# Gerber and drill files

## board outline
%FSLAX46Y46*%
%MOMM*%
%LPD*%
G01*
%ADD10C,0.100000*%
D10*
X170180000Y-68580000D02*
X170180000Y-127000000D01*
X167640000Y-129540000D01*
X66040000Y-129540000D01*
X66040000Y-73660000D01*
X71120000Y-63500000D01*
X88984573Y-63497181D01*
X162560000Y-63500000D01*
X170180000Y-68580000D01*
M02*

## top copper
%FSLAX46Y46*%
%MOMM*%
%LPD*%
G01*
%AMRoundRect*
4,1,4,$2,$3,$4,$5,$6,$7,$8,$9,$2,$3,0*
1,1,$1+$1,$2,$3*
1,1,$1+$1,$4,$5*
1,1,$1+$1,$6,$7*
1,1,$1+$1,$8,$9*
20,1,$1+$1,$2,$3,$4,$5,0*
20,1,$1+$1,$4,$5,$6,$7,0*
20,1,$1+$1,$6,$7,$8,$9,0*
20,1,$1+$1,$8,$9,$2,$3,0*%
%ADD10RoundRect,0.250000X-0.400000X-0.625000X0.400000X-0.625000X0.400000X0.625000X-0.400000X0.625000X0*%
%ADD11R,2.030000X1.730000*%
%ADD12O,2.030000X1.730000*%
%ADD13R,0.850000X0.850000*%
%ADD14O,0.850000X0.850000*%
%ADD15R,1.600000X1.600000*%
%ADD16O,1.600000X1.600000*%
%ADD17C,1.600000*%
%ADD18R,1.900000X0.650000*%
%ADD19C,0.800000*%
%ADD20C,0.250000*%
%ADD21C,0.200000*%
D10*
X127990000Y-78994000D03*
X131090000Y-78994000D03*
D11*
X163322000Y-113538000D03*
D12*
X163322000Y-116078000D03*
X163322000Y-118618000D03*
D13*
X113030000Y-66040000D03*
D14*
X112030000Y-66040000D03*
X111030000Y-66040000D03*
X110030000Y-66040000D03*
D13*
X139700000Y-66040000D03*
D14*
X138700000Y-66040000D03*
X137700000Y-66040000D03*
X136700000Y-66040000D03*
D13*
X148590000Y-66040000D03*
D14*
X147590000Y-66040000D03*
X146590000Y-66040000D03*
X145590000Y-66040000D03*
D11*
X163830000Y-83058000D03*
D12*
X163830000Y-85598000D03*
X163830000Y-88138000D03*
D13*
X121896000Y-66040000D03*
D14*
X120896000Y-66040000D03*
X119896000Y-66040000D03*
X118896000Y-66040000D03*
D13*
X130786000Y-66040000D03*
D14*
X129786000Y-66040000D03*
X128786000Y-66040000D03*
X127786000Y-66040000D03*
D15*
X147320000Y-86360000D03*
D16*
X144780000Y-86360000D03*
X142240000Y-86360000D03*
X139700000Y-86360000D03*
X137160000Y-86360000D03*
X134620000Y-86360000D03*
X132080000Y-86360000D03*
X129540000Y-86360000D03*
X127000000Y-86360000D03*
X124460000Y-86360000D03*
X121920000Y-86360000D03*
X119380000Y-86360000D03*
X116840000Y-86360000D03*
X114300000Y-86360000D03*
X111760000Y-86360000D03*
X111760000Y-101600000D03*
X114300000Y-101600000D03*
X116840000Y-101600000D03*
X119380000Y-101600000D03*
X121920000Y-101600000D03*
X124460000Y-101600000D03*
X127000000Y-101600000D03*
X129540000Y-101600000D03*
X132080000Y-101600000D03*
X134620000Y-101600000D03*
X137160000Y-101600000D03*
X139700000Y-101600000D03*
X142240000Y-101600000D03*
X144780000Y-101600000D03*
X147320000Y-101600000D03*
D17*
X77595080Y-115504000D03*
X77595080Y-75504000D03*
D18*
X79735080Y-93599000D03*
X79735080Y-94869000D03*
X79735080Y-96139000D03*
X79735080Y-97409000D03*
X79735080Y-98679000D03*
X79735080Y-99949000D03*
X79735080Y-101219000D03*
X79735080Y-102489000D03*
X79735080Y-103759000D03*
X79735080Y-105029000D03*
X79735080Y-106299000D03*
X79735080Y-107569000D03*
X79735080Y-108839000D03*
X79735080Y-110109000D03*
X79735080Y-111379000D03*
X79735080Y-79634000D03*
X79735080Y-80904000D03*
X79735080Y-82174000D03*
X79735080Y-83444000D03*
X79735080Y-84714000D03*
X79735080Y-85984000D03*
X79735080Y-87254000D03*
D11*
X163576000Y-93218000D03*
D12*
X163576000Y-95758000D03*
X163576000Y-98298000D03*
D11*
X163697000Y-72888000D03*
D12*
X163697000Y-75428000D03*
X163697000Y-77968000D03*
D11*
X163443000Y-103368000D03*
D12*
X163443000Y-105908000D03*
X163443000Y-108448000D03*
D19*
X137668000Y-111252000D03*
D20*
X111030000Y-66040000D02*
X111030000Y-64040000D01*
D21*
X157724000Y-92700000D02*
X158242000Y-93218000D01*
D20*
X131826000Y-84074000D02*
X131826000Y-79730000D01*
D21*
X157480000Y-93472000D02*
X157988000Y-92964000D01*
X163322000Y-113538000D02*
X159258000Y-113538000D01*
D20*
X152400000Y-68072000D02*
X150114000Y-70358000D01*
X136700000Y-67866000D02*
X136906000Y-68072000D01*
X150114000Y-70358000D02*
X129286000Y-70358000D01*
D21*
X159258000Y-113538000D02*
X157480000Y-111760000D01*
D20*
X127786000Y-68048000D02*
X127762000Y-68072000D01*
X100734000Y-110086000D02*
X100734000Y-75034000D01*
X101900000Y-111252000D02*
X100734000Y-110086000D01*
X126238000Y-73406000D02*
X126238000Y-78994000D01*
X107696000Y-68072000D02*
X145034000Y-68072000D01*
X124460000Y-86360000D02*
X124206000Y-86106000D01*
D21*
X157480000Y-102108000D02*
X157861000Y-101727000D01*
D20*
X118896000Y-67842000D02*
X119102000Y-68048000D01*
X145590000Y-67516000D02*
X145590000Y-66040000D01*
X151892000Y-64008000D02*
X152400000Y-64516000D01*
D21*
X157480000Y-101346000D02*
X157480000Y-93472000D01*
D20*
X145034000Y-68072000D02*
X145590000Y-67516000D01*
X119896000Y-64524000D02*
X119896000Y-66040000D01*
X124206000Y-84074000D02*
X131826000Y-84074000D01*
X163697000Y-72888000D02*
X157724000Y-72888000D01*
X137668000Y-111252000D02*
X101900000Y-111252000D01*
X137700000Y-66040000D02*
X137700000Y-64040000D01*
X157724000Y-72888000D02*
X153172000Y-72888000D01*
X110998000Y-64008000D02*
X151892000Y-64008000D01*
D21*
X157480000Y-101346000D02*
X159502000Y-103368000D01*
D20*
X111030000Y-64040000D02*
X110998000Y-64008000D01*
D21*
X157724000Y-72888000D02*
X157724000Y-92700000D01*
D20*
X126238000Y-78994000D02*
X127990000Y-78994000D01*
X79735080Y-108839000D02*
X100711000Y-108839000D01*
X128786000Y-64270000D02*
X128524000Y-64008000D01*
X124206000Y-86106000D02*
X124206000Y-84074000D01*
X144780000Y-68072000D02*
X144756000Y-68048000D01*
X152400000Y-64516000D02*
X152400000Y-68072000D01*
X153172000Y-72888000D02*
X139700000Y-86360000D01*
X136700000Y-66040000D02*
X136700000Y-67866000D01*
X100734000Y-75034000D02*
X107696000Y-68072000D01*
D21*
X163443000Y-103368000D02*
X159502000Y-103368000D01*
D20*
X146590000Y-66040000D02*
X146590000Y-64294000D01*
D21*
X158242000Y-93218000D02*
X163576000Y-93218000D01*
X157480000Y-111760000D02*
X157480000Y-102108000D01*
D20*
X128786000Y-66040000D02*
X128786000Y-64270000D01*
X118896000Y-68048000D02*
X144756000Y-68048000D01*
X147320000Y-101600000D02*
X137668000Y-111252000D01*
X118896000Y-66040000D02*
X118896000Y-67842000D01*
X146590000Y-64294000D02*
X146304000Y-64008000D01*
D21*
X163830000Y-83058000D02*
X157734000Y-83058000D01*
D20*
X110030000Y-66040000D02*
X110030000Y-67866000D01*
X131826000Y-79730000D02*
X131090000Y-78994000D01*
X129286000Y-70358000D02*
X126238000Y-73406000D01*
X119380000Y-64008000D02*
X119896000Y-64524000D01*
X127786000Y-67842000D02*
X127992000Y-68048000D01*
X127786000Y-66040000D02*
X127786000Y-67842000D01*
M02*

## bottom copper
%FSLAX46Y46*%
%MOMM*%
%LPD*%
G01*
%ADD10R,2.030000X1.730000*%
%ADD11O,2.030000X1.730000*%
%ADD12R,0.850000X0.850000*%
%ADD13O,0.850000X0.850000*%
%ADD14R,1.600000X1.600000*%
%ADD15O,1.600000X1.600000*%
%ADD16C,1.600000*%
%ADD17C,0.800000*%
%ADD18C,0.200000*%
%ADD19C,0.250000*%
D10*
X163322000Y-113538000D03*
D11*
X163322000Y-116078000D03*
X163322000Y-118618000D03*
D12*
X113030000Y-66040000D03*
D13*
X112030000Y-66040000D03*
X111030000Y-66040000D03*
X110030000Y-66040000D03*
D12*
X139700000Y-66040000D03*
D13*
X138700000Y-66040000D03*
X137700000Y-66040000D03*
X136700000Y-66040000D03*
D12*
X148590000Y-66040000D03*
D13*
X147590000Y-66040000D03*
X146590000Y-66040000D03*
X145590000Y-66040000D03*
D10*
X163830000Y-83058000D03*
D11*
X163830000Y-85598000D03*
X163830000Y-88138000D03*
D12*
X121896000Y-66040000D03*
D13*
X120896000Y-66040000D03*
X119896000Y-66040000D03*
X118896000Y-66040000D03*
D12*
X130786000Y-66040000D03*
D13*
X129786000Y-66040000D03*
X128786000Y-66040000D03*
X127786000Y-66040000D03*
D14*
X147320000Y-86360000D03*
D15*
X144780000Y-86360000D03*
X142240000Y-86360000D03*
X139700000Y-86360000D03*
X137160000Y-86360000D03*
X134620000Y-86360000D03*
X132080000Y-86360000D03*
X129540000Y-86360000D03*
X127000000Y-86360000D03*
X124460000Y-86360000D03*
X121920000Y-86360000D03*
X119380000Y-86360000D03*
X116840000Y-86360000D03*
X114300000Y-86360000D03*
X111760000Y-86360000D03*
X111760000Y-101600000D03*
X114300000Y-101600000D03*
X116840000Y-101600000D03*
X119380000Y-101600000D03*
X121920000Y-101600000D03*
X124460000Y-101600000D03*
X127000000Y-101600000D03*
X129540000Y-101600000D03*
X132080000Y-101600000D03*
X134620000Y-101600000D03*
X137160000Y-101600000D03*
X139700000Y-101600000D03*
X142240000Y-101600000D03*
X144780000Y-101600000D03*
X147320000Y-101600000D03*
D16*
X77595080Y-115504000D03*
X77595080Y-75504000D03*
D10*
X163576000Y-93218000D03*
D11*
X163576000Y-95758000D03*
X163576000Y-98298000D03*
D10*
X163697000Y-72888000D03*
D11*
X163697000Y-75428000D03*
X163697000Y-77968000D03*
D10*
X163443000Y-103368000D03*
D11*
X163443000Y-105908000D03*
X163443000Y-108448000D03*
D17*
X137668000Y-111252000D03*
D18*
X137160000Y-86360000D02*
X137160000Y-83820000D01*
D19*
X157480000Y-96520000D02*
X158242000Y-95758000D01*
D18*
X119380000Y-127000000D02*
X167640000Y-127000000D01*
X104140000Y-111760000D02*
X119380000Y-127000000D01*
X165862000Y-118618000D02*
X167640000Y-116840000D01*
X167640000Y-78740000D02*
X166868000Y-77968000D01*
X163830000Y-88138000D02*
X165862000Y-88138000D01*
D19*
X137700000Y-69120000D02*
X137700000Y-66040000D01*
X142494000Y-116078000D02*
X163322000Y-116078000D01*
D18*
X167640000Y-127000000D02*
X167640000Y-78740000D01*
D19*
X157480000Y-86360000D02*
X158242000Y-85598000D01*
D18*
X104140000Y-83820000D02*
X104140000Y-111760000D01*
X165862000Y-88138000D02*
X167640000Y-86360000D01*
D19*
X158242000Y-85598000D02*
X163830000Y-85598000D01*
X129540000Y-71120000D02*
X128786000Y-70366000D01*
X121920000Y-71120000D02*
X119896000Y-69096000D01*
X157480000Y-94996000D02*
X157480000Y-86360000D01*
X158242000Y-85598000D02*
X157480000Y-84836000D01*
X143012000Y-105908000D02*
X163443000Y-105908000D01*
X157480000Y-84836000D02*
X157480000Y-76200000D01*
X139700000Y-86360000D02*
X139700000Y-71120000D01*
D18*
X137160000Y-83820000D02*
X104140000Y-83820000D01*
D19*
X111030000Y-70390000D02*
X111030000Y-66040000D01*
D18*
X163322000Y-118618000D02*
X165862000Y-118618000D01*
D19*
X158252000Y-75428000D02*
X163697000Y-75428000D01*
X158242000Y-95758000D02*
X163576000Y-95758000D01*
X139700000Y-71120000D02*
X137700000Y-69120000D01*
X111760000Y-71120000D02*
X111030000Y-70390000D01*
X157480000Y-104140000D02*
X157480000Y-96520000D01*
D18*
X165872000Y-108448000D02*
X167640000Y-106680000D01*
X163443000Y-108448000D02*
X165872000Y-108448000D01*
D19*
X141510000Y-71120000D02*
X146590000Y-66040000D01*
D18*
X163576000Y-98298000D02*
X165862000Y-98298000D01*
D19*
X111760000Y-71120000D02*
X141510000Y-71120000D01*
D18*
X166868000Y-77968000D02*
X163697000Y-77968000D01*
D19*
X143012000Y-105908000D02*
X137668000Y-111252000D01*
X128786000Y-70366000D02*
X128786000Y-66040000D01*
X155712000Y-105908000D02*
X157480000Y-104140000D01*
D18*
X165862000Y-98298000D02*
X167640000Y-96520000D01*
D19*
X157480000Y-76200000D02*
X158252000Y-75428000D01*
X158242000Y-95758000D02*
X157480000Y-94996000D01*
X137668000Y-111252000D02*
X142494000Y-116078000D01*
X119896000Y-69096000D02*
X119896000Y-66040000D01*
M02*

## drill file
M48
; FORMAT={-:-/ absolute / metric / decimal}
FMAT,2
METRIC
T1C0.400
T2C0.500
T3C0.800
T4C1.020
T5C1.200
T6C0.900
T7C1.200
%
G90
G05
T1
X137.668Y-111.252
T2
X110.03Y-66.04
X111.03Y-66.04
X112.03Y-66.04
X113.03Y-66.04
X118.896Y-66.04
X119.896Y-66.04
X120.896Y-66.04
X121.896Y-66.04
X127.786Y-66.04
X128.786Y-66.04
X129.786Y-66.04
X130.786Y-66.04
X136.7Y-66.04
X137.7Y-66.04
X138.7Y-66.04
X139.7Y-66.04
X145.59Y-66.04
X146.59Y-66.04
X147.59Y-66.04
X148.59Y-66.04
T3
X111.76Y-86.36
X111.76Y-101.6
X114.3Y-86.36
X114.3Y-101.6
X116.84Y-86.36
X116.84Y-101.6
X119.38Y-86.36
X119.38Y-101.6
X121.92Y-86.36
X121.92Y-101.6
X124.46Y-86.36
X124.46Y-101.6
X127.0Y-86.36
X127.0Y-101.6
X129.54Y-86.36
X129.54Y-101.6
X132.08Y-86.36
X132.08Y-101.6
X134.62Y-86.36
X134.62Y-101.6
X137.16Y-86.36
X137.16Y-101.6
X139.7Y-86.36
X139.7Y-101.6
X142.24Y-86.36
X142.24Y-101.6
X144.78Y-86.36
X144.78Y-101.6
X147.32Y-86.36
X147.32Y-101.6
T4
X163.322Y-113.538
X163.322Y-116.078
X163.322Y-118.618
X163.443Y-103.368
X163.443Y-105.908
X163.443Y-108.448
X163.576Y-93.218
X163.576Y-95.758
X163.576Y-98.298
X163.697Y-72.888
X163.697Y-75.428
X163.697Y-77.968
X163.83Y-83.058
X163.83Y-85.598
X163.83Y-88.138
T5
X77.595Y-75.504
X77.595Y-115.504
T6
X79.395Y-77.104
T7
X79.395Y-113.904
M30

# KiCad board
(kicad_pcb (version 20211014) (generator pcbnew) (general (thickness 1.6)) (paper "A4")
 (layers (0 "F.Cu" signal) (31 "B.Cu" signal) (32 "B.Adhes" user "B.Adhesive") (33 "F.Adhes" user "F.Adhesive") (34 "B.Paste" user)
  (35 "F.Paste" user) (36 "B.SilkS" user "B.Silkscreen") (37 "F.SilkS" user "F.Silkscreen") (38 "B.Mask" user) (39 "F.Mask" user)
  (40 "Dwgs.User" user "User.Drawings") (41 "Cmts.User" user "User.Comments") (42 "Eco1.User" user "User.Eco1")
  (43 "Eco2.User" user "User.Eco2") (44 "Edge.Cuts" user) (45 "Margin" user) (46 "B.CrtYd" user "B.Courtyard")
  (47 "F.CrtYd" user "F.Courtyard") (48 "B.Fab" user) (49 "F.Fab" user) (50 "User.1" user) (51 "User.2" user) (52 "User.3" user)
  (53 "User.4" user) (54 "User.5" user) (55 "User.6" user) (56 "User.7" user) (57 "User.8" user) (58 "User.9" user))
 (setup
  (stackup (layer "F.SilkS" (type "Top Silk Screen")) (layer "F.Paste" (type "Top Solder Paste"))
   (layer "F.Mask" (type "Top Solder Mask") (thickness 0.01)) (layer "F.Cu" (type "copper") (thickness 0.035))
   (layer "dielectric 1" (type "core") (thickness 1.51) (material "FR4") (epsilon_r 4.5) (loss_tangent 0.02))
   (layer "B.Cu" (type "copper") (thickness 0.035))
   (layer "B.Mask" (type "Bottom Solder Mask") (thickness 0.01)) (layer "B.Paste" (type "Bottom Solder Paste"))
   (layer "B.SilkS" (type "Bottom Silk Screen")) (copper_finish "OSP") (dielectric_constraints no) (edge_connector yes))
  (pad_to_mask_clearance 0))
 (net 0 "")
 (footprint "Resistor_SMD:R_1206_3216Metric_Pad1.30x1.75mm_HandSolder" (layer "F.Cu") (at 129.54 78.994)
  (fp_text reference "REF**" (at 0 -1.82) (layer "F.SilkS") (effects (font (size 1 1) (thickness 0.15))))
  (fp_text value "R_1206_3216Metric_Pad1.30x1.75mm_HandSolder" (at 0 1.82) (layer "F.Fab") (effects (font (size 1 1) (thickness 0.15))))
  (pad "1" smd roundrect (at -1.55 0) (size 1.3 1.75) (layers "F.Cu" "F.Paste" "F.Mask") (roundrect_rratio 0.1923076923))
  (pad "2" smd roundrect (at 1.55 0) (size 1.3 1.75) (layers "F.Cu" "F.Paste" "F.Mask") (roundrect_rratio 0.1923076923)))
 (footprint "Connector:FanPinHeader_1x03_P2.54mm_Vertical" (layer "F.Cu") (at 163.322 113.538 -90)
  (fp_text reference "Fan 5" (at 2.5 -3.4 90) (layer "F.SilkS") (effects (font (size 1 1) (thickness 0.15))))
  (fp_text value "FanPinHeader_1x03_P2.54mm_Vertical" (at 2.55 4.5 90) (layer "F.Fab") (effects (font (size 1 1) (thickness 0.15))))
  (pad "1" thru_hole rect (at 0 0) (size 2.03 1.73) (drill 1.02) (layers *.Cu *.Mask))
  (pad "2" thru_hole oval (at 2.54 0) (size 2.03 1.73) (drill 1.02) (layers *.Cu *.Mask))
  (pad "3" thru_hole oval (at 5.08 0) (size 2.03 1.73) (drill 1.02) (layers *.Cu *.Mask)))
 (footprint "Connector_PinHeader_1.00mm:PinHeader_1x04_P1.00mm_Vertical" (layer "F.Cu") (at 113.03 66.04 -90)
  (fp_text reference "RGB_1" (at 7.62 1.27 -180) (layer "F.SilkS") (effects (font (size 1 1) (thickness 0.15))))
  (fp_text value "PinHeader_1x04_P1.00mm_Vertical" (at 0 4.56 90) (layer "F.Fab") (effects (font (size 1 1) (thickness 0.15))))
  (pad "1" thru_hole rect (at 0 0 270) (size 0.85 0.85) (drill 0.5) (layers *.Cu *.Mask))
  (pad "2" thru_hole oval (at 0 1 270) (size 0.85 0.85) (drill 0.5) (layers *.Cu *.Mask))
  (pad "3" thru_hole oval (at 0 2 270) (size 0.85 0.85) (drill 0.5) (layers *.Cu *.Mask))
  (pad "4" thru_hole oval (at 0 3 270) (size 0.85 0.85) (drill 0.5) (layers *.Cu *.Mask)))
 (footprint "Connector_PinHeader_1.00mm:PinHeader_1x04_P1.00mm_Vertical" (layer "F.Cu") (at 139.7 66.04 -90)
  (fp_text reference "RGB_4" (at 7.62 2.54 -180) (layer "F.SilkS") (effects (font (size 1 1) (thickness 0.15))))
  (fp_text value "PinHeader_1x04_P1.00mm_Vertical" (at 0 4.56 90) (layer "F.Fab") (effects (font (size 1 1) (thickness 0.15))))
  (pad "1" thru_hole rect (at 0 0 270) (size 0.85 0.85) (drill 0.5) (layers *.Cu *.Mask))
  (pad "2" thru_hole oval (at 0 1 270) (size 0.85 0.85) (drill 0.5) (layers *.Cu *.Mask))
  (pad "3" thru_hole oval (at 0 2 270) (size 0.85 0.85) (drill 0.5) (layers *.Cu *.Mask))
  (pad "4" thru_hole oval (at 0 3 270) (size 0.85 0.85) (drill 0.5) (layers *.Cu *.Mask)))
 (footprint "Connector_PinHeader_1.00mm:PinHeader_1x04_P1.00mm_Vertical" (layer "F.Cu") (at 148.59 66.04 -90)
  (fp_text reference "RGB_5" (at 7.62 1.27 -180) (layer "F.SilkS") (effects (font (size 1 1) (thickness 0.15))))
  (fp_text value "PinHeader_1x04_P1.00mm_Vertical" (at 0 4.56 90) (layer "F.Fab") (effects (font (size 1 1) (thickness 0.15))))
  (pad "1" thru_hole rect (at 0 0 270) (size 0.85 0.85) (drill 0.5) (layers *.Cu *.Mask))
  (pad "2" thru_hole oval (at 0 1 270) (size 0.85 0.85) (drill 0.5) (layers *.Cu *.Mask))
  (pad "3" thru_hole oval (at 0 2 270) (size 0.85 0.85) (drill 0.5) (layers *.Cu *.Mask))
  (pad "4" thru_hole oval (at 0 3 270) (size 0.85 0.85) (drill 0.5) (layers *.Cu *.Mask)))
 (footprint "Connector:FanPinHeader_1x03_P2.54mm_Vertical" (layer "F.Cu") (at 163.83 83.058 -90)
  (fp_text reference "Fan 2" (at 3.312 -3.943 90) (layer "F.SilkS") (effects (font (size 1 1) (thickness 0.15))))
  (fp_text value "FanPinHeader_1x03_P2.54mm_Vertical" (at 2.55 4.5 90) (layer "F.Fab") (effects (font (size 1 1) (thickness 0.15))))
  (pad "1" thru_hole rect (at 0 0) (size 2.03 1.73) (drill 1.02) (layers *.Cu *.Mask))
  (pad "2" thru_hole oval (at 2.54 0) (size 2.03 1.73) (drill 1.02) (layers *.Cu *.Mask))
  (pad "3" thru_hole oval (at 5.08 0) (size 2.03 1.73) (drill 1.02) (layers *.Cu *.Mask)))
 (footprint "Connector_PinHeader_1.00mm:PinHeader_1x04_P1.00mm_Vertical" (layer "F.Cu") (at 121.896 66.04 -90)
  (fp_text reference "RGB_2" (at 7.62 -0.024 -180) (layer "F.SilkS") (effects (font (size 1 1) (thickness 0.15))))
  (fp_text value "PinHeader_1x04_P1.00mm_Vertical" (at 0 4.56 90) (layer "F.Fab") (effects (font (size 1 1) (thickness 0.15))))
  (pad "1" thru_hole rect (at 0 0 270) (size 0.85 0.85) (drill 0.5) (layers *.Cu *.Mask))
  (pad "2" thru_hole oval (at 0 1 270) (size 0.85 0.85) (drill 0.5) (layers *.Cu *.Mask))
  (pad "3" thru_hole oval (at 0 2 270) (size 0.85 0.85) (drill 0.5) (layers *.Cu *.Mask))
  (pad "4" thru_hole oval (at 0 3 270) (size 0.85 0.85) (drill 0.5) (layers *.Cu *.Mask)))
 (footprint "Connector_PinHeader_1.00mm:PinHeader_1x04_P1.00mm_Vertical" (layer "F.Cu") (at 130.786 66.04 -90)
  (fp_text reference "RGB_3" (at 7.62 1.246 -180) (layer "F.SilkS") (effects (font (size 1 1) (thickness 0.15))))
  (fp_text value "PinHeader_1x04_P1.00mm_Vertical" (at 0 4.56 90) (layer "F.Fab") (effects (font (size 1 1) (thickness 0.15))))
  (pad "1" thru_hole rect (at 0 0 270) (size 0.85 0.85) (drill 0.5) (layers *.Cu *.Mask))
  (pad "2" thru_hole oval (at 0 1 270) (size 0.85 0.85) (drill 0.5) (layers *.Cu *.Mask))
  (pad "3" thru_hole oval (at 0 2 270) (size 0.85 0.85) (drill 0.5) (layers *.Cu *.Mask))
  (pad "4" thru_hole oval (at 0 3 270) (size 0.85 0.85) (drill 0.5) (layers *.Cu *.Mask)))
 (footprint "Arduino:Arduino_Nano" (layer "F.Cu") (at 147.32 86.36 -90)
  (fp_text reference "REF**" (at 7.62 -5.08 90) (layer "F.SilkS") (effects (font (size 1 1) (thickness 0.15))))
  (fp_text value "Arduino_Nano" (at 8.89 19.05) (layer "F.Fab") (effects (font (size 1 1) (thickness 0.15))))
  (pad "1" thru_hole rect locked (at 0 0 270) (size 1.6 1.6) (drill 0.8) (layers *.Cu *.Mask))
  (pad "2" thru_hole oval locked (at 0 2.54 270) (size 1.6 1.6) (drill 0.8) (layers *.Cu *.Mask))
  (pad "3" thru_hole oval locked (at 0 5.08 270) (size 1.6 1.6) (drill 0.8) (layers *.Cu *.Mask))
  (pad "4" thru_hole oval locked (at 0 7.62 270) (size 1.6 1.6) (drill 0.8) (layers *.Cu *.Mask))
  (pad "5" thru_hole oval locked (at 0 10.16 270) (size 1.6 1.6) (drill 0.8) (layers *.Cu *.Mask))
  (pad "6" thru_hole oval locked (at 0 12.7 270) (size 1.6 1.6) (drill 0.8) (layers *.Cu *.Mask))
  (pad "7" thru_hole oval locked (at 0 15.24 270) (size 1.6 1.6) (drill 0.8) (layers *.Cu *.Mask))
  (pad "8" thru_hole oval locked (at 0 17.78 270) (size 1.6 1.6) (drill 0.8) (layers *.Cu *.Mask))
  (pad "9" thru_hole oval locked (at 0 20.32 270) (size 1.6 1.6) (drill 0.8) (layers *.Cu *.Mask))
  (pad "10" thru_hole oval locked (at 0 22.86 270) (size 1.6 1.6) (drill 0.8) (layers *.Cu *.Mask))
  (pad "11" thru_hole oval locked (at 0 25.4 270) (size 1.6 1.6) (drill 0.8) (layers *.Cu *.Mask))
  (pad "12" thru_hole oval locked (at 0 27.94 270) (size 1.6 1.6) (drill 0.8) (layers *.Cu *.Mask))
  (pad "13" thru_hole oval locked (at 0 30.48 270) (size 1.6 1.6) (drill 0.8) (layers *.Cu *.Mask))
  (pad "14" thru_hole oval locked (at 0 33.02 270) (size 1.6 1.6) (drill 0.8) (layers *.Cu *.Mask))
  (pad "15" thru_hole oval locked (at 0 35.56 270) (size 1.6 1.6) (drill 0.8) (layers *.Cu *.Mask))
  (pad "16" thru_hole oval locked (at 15.24 35.56 270) (size 1.6 1.6) (drill 0.8) (layers *.Cu *.Mask))
  (pad "17" thru_hole oval locked (at 15.24 33.02 270) (size 1.6 1.6) (drill 0.8) (layers *.Cu *.Mask))
  (pad "18" thru_hole oval locked (at 15.24 30.48 270) (size 1.6 1.6) (drill 0.8) (layers *.Cu *.Mask))
  (pad "19" thru_hole oval locked (at 15.24 27.94 270) (size 1.6 1.6) (drill 0.8) (layers *.Cu *.Mask))
  (pad "20" thru_hole oval locked (at 15.24 25.4 270) (size 1.6 1.6) (drill 0.8) (layers *.Cu *.Mask))
  (pad "21" thru_hole oval locked (at 15.24 22.86 270) (size 1.6 1.6) (drill 0.8) (layers *.Cu *.Mask))
  (pad "22" thru_hole oval locked (at 15.24 20.32 270) (size 1.6 1.6) (drill 0.8) (layers *.Cu *.Mask))
  (pad "23" thru_hole oval locked (at 15.24 17.78 270) (size 1.6 1.6) (drill 0.8) (layers *.Cu *.Mask))
  (pad "24" thru_hole oval locked (at 15.24 15.24 270) (size 1.6 1.6) (drill 0.8) (layers *.Cu *.Mask))
  (pad "25" thru_hole oval locked (at 15.24 12.7 270) (size 1.6 1.6) (drill 0.8) (layers *.Cu *.Mask))
  (pad "26" thru_hole oval locked (at 15.24 10.16 270) (size 1.6 1.6) (drill 0.8) (layers *.Cu *.Mask))
  (pad "27" thru_hole oval locked (at 15.24 7.62 270) (size 1.6 1.6) (drill 0.8) (layers *.Cu *.Mask))
  (pad "28" thru_hole oval locked (at 15.24 5.08 270) (size 1.6 1.6) (drill 0.8) (layers *.Cu *.Mask))
  (pad "29" thru_hole oval locked (at 15.24 2.54 270) (size 1.6 1.6) (drill 0.8) (layers *.Cu *.Mask))
  (pad "30" thru_hole oval locked (at 15.24 0 270) (size 1.6 1.6) (drill 0.8) (layers *.Cu *.Mask)))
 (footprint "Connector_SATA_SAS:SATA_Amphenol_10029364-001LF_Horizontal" (layer "F.Cu") (at 78.74 95.504 90)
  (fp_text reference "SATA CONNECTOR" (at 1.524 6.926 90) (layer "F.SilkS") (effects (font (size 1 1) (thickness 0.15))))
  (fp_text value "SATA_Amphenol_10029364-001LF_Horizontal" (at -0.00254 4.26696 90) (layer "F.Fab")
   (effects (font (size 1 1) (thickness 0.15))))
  (pad "" np_thru_hole circle (at -18.4 0.65508 90) (size 1.2 1.2) (drill 1.2) (layers *.Mask "B.Cu"))
  (pad "" np_thru_hole circle (at 18.4 0.65508 90) (size 0.9 0.9) (drill 0.9) (layers *.Mask "B.Cu"))
  (pad "MP" thru_hole circle (at -20 -1.14492 90) (size 1.6 1.6) (drill 1.2) (layers *.Cu *.Mask) (zone_connect 2))
  (pad "MP" thru_hole circle (at 20 -1.14492 90) (size 1.6 1.6) (drill 1.2) (layers *.Cu *.Mask))
  (pad "P1" smd rect (at 1.905 0.99508 90) (size 0.65 1.9) (layers "F.Cu" "F.Paste" "F.Mask"))
  (pad "P2" smd rect (at 0.635 0.99508 90) (size 0.65 1.9) (layers "F.Cu" "F.Paste" "F.Mask"))
  (pad "P3" smd rect (at -0.635 0.99508 90) (size 0.65 1.9) (layers "F.Cu" "F.Paste" "F.Mask"))
  (pad "P4" smd rect (at -1.905 0.99508 90) (size 0.65 1.9) (layers "F.Cu" "F.Paste" "F.Mask"))
  (pad "P5" smd rect (at -3.175 0.99508 90) (size 0.65 1.9) (layers "F.Cu" "F.Paste" "F.Mask"))
  (pad "P6" smd rect (at -4.445 0.99508 90) (size 0.65 1.9) (layers "F.Cu" "F.Paste" "F.Mask"))
  (pad "P7" smd rect (at -5.715 0.99508 90) (size 0.65 1.9) (layers "F.Cu" "F.Paste" "F.Mask"))
  (pad "P8" smd rect (at -6.985 0.99508 90) (size 0.65 1.9) (layers "F.Cu" "F.Paste" "F.Mask"))
  (pad "P9" smd rect (at -8.255 0.99508 90) (size 0.65 1.9) (layers "F.Cu" "F.Paste" "F.Mask"))
  (pad "P10" smd rect (at -9.525 0.99508 90) (size 0.65 1.9) (layers "F.Cu" "F.Paste" "F.Mask"))
  (pad "P11" smd rect (at -10.795 0.99508 90) (size 0.65 1.9) (layers "F.Cu" "F.Paste" "F.Mask"))
  (pad "P12" smd rect (at -12.065 0.99508 90) (size 0.65 1.9) (layers "F.Cu" "F.Paste" "F.Mask"))
  (pad "P13" smd rect (at -13.335 0.99508 90) (size 0.65 1.9) (layers "F.Cu" "F.Paste" "F.Mask"))
  (pad "P14" smd rect (at -14.605 0.99508 90) (size 0.65 1.9) (layers "F.Cu" "F.Paste" "F.Mask"))
  (pad "P15" smd rect (at -15.875 0.99508 90) (size 0.65 1.9) (layers "F.Cu" "F.Paste" "F.Mask"))
  (pad "S1" smd rect (at 15.87 0.99508 90) (size 0.65 1.9) (layers "F.Cu" "F.Paste" "F.Mask"))
  (pad "S2" smd rect (at 14.6 0.99508 90) (size 0.65 1.9) (layers "F.Cu" "F.Paste" "F.Mask"))
  (pad "S3" smd rect (at 13.33 0.99508 90) (size 0.65 1.9) (layers "F.Cu" "F.Paste" "F.Mask"))
  (pad "S4" smd rect (at 12.06 0.99508 90) (size 0.65 1.9) (layers "F.Cu" "F.Paste" "F.Mask"))
  (pad "S5" smd rect (at 10.79 0.99508 90) (size 0.65 1.9) (layers "F.Cu" "F.Paste" "F.Mask"))
  (pad "S6" smd rect (at 9.52 0.99508 90) (size 0.65 1.9) (layers "F.Cu" "F.Paste" "F.Mask"))
  (pad "S7" smd rect (at 8.25 0.99508 90) (size 0.65 1.9) (layers "F.Cu" "F.Paste" "F.Mask")))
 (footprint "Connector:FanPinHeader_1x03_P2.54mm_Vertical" (layer "F.Cu") (at 163.576 93.218 -90)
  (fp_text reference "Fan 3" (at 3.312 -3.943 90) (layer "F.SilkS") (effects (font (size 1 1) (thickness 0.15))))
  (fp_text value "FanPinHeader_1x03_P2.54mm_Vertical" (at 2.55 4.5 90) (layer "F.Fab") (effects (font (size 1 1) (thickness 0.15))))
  (pad "1" thru_hole rect (at 0 0) (size 2.03 1.73) (drill 1.02) (layers *.Cu *.Mask))
  (pad "2" thru_hole oval (at 2.54 0) (size 2.03 1.73) (drill 1.02) (layers *.Cu *.Mask))
  (pad "3" thru_hole oval (at 5.08 0) (size 2.03 1.73) (drill 1.02) (layers *.Cu *.Mask)))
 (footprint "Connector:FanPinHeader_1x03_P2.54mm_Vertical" (layer "F.Cu") (at 163.697 72.888 -90)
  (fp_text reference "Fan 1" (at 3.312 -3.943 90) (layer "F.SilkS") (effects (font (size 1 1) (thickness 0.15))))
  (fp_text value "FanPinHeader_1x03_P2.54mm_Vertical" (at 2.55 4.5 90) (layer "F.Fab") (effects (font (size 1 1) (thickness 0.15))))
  (pad "1" thru_hole rect (at 0 0) (size 2.03 1.73) (drill 1.02) (layers *.Cu *.Mask))
  (pad "2" thru_hole oval (at 2.54 0) (size 2.03 1.73) (drill 1.02) (layers *.Cu *.Mask))
  (pad "3" thru_hole oval (at 5.08 0) (size 2.03 1.73) (drill 1.02) (layers *.Cu *.Mask)))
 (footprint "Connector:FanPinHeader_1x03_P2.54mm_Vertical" (layer "F.Cu") (at 163.443 103.368 -90)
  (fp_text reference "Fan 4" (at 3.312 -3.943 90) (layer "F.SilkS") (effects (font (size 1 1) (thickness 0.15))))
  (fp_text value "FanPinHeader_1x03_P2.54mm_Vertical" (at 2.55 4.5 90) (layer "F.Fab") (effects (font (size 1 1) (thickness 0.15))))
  (pad "1" thru_hole rect (at 0 0) (size 2.03 1.73) (drill 1.02) (layers *.Cu *.Mask))
  (pad "2" thru_hole oval (at 2.54 0) (size 2.03 1.73) (drill 1.02) (layers *.Cu *.Mask))
  (pad "3" thru_hole oval (at 5.08 0) (size 2.03 1.73) (drill 1.02) (layers *.Cu *.Mask)))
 (gr_poly
  (pts (xy 170.18 68.58) (xy 170.18 127) (xy 167.64 129.54) (xy 66.04 129.54) (xy 66.04 73.66) (xy 71.12 63.5) (xy 88.984573 63.497181)
   (xy 162.56 63.5))
  (layer "Edge.Cuts") (width 0.1) (fill none))
 (segment (start 111.03 66.04) (end 111.03 64.04) (width 0.25) (layer "F.Cu") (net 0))
 (segment (start 157.724 92.7) (end 158.242 93.218) (width 0.2) (layer "F.Cu") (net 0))
 (segment (start 131.826 84.074) (end 131.826 79.73) (width 0.25) (layer "F.Cu") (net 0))
 (segment (start 157.48 93.472) (end 157.988 92.964) (width 0.2) (layer "F.Cu") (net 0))
 (segment (start 163.322 113.538) (end 159.258 113.538) (width 0.2) (layer "F.Cu") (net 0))
 (segment (start 152.4 68.072) (end 150.114 70.358) (width 0.25) (layer "F.Cu") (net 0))
 (segment (start 136.7 67.866) (end 136.906 68.072) (width 0.25) (layer "F.Cu") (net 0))
 (segment (start 150.114 70.358) (end 129.286 70.358) (width 0.25) (layer "F.Cu") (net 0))
 (segment (start 159.258 113.538) (end 157.48 111.76) (width 0.2) (layer "F.Cu") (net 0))
 (segment (start 127.786 68.048) (end 127.762 68.072) (width 0.25) (layer "F.Cu") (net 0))
 (segment (start 100.734 110.086) (end 100.734 75.034) (width 0.25) (layer "F.Cu") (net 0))
 (segment (start 101.9 111.252) (end 100.734 110.086) (width 0.25) (layer "F.Cu") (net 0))
 (segment (start 126.238 73.406) (end 126.238 78.994) (width 0.25) (layer "F.Cu") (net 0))
 (segment (start 107.696 68.072) (end 145.034 68.072) (width 0.25) (layer "F.Cu") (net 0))
 (segment (start 124.46 86.36) (end 124.206 86.106) (width 0.25) (layer "F.Cu") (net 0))
 (segment (start 157.48 102.108) (end 157.861 101.727) (width 0.2) (layer "F.Cu") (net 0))
 (segment (start 118.896 67.842) (end 119.102 68.048) (width 0.25) (layer "F.Cu") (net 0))
 (segment (start 145.59 67.516) (end 145.59 66.04) (width 0.25) (layer "F.Cu") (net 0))
 (segment (start 151.892 64.008) (end 152.4 64.516) (width 0.25) (layer "F.Cu") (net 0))
 (segment (start 157.48 101.346) (end 157.48 93.472) (width 0.2) (layer "F.Cu") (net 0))
 (segment (start 145.034 68.072) (end 145.59 67.516) (width 0.25) (layer "F.Cu") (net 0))
 (segment (start 119.896 64.524) (end 119.896 66.04) (width 0.25) (layer "F.Cu") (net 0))
 (segment (start 124.206 84.074) (end 131.826 84.074) (width 0.25) (layer "F.Cu") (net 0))
 (segment (start 163.697 72.888) (end 157.724 72.888) (width 0.25) (layer "F.Cu") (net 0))
 (segment (start 137.668 111.252) (end 101.9 111.252) (width 0.25) (layer "F.Cu") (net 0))
 (segment (start 137.7 66.04) (end 137.7 64.04) (width 0.25) (layer "F.Cu") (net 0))
 (segment (start 157.724 72.888) (end 153.172 72.888) (width 0.25) (layer "F.Cu") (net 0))
 (segment (start 110.998 64.008) (end 151.892 64.008) (width 0.25) (layer "F.Cu") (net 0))
 (segment (start 157.48 101.346) (end 159.502 103.368) (width 0.2) (layer "F.Cu") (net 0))
 (segment (start 111.03 64.04) (end 110.998 64.008) (width 0.25) (layer "F.Cu") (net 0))
 (segment (start 157.724 72.888) (end 157.724 92.7) (width 0.2) (layer "F.Cu") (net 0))
 (segment (start 126.238 78.994) (end 127.99 78.994) (width 0.25) (layer "F.Cu") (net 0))
 (segment (start 79.73508 108.839) (end 100.711 108.839) (width 0.25) (layer "F.Cu") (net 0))
 (segment (start 128.786 64.27) (end 128.524 64.008) (width 0.25) (layer "F.Cu") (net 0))
 (segment (start 124.206 86.106) (end 124.206 84.074) (width 0.25) (layer "F.Cu") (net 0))
 (segment (start 144.78 68.072) (end 144.756 68.048) (width 0.25) (layer "F.Cu") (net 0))
 (segment (start 152.4 64.516) (end 152.4 68.072) (width 0.25) (layer "F.Cu") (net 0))
 (segment (start 153.172 72.888) (end 139.7 86.36) (width 0.25) (layer "F.Cu") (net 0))
 (segment (start 136.7 66.04) (end 136.7 67.866) (width 0.25) (layer "F.Cu") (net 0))
 (segment (start 100.734 75.034) (end 107.696 68.072) (width 0.25) (layer "F.Cu") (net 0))
 (segment (start 163.443 103.368) (end 159.502 103.368) (width 0.2) (layer "F.Cu") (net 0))
 (segment (start 146.59 66.04) (end 146.59 64.294) (width 0.25) (layer "F.Cu") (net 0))
 (segment (start 158.242 93.218) (end 163.576 93.218) (width 0.2) (layer "F.Cu") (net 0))
 (segment (start 157.48 111.76) (end 157.48 102.108) (width 0.2) (layer "F.Cu") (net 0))
 (segment (start 128.786 66.04) (end 128.786 64.27) (width 0.25) (layer "F.Cu") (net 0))
 (segment (start 118.896 68.048) (end 144.756 68.048) (width 0.25) (layer "F.Cu") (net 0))
 (segment (start 147.32 101.6) (end 137.668 111.252) (width 0.25) (layer "F.Cu") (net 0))
 (segment (start 118.896 66.04) (end 118.896 67.842) (width 0.25) (layer "F.Cu") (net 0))
 (segment (start 146.59 64.294) (end 146.304 64.008) (width 0.25) (layer "F.Cu") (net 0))
 (segment (start 163.83 83.058) (end 157.734 83.058) (width 0.2) (layer "F.Cu") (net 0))
 (segment (start 110.03 66.04) (end 110.03 67.866) (width 0.25) (layer "F.Cu") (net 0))
 (segment (start 131.826 79.73) (end 131.09 78.994) (width 0.25) (layer "F.Cu") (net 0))
 (segment (start 129.286 70.358) (end 126.238 73.406) (width 0.25) (layer "F.Cu") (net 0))
 (segment (start 119.38 64.008) (end 119.896 64.524) (width 0.25) (layer "F.Cu") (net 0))
 (segment (start 127.786 67.842) (end 127.992 68.048) (width 0.25) (layer "F.Cu") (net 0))
 (segment (start 127.786 66.04) (end 127.786 67.842) (width 0.25) (layer "F.Cu") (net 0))
 (via blind (at 137.668 111.252) (size 0.8) (drill 0.4) (layers "F.Cu" "B.Cu") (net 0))
 (segment (start 137.16 86.36) (end 137.16 83.82) (width 0.2) (layer "B.Cu") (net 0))
 (segment (start 157.48 96.52) (end 158.242 95.758) (width 0.25) (layer "B.Cu") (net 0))
 (segment (start 119.38 127) (end 167.64 127) (width 0.2) (layer "B.Cu") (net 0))
 (segment (start 104.14 111.76) (end 119.38 127) (width 0.2) (layer "B.Cu") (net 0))
 (segment (start 165.862 118.618) (end 167.64 116.84) (width 0.2) (layer "B.Cu") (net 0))
 (segment (start 167.64 78.74) (end 166.868 77.968) (width 0.2) (layer "B.Cu") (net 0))
 (segment (start 163.83 88.138) (end 165.862 88.138) (width 0.2) (layer "B.Cu") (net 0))
 (segment (start 137.7 69.12) (end 137.7 66.04) (width 0.25) (layer "B.Cu") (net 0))
 (segment (start 142.494 116.078) (end 163.322 116.078) (width 0.25) (layer "B.Cu") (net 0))
 (segment (start 167.64 127) (end 167.64 78.74) (width 0.2) (layer "B.Cu") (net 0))
 (segment (start 157.48 86.36) (end 158.242 85.598) (width 0.25) (layer "B.Cu") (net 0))
 (segment (start 104.14 83.82) (end 104.14 111.76) (width 0.2) (layer "B.Cu") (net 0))
 (segment (start 165.862 88.138) (end 167.64 86.36) (width 0.2) (layer "B.Cu") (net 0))
 (segment (start 158.242 85.598) (end 163.83 85.598) (width 0.25) (layer "B.Cu") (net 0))
 (segment (start 129.54 71.12) (end 128.786 70.366) (width 0.25) (layer "B.Cu") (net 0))
 (segment (start 121.92 71.12) (end 119.896 69.096) (width 0.25) (layer "B.Cu") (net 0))
 (segment (start 157.48 94.996) (end 157.48 86.36) (width 0.25) (layer "B.Cu") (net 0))
 (segment (start 158.242 85.598) (end 157.48 84.836) (width 0.25) (layer "B.Cu") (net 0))
 (segment (start 143.012 105.908) (end 163.443 105.908) (width 0.25) (layer "B.Cu") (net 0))
 (segment (start 157.48 84.836) (end 157.48 76.2) (width 0.25) (layer "B.Cu") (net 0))
 (segment (start 139.7 86.36) (end 139.7 71.12) (width 0.25) (layer "B.Cu") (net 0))
 (segment (start 137.16 83.82) (end 104.14 83.82) (width 0.2) (layer "B.Cu") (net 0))
 (segment (start 111.03 70.39) (end 111.03 66.04) (width 0.25) (layer "B.Cu") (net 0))
 (segment (start 163.322 118.618) (end 165.862 118.618) (width 0.2) (layer "B.Cu") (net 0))
 (segment (start 158.252 75.428) (end 163.697 75.428) (width 0.25) (layer "B.Cu") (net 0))
 (segment (start 158.242 95.758) (end 163.576 95.758) (width 0.25) (layer "B.Cu") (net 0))
 (segment (start 139.7 71.12) (end 137.7 69.12) (width 0.25) (layer "B.Cu") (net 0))
 (segment (start 111.76 71.12) (end 111.03 70.39) (width 0.25) (layer "B.Cu") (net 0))
 (segment (start 157.48 104.14) (end 157.48 96.52) (width 0.25) (layer "B.Cu") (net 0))
 (segment (start 165.872 108.448) (end 167.64 106.68) (width 0.2) (layer "B.Cu") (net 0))
 (segment (start 163.443 108.448) (end 165.872 108.448) (width 0.2) (layer "B.Cu") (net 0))
 (segment (start 141.51 71.12) (end 146.59 66.04) (width 0.25) (layer "B.Cu") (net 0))
 (segment (start 163.576 98.298) (end 165.862 98.298) (width 0.2) (layer "B.Cu") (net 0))
 (segment (start 111.76 71.12) (end 141.51 71.12) (width 0.25) (layer "B.Cu") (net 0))
 (segment (start 166.868 77.968) (end 163.697 77.968) (width 0.2) (layer "B.Cu") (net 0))
 (segment (start 143.012 105.908) (end 137.668 111.252) (width 0.25) (layer "B.Cu") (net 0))
 (segment (start 128.786 70.366) (end 128.786 66.04) (width 0.25) (layer "B.Cu") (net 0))
 (segment (start 155.712 105.908) (end 157.48 104.14) (width 0.25) (layer "B.Cu") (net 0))
 (segment (start 165.862 98.298) (end 167.64 96.52) (width 0.2) (layer "B.Cu") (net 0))
 (segment (start 157.48 76.2) (end 158.252 75.428) (width 0.25) (layer "B.Cu") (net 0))
 (segment (start 158.242 95.758) (end 157.48 94.996) (width 0.25) (layer "B.Cu") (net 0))
 (segment (start 137.668 111.252) (end 142.494 116.078) (width 0.25) (layer "B.Cu") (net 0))
 (segment (start 119.896 69.096) (end 119.896 66.04) (width 0.25) (layer "B.Cu") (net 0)))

